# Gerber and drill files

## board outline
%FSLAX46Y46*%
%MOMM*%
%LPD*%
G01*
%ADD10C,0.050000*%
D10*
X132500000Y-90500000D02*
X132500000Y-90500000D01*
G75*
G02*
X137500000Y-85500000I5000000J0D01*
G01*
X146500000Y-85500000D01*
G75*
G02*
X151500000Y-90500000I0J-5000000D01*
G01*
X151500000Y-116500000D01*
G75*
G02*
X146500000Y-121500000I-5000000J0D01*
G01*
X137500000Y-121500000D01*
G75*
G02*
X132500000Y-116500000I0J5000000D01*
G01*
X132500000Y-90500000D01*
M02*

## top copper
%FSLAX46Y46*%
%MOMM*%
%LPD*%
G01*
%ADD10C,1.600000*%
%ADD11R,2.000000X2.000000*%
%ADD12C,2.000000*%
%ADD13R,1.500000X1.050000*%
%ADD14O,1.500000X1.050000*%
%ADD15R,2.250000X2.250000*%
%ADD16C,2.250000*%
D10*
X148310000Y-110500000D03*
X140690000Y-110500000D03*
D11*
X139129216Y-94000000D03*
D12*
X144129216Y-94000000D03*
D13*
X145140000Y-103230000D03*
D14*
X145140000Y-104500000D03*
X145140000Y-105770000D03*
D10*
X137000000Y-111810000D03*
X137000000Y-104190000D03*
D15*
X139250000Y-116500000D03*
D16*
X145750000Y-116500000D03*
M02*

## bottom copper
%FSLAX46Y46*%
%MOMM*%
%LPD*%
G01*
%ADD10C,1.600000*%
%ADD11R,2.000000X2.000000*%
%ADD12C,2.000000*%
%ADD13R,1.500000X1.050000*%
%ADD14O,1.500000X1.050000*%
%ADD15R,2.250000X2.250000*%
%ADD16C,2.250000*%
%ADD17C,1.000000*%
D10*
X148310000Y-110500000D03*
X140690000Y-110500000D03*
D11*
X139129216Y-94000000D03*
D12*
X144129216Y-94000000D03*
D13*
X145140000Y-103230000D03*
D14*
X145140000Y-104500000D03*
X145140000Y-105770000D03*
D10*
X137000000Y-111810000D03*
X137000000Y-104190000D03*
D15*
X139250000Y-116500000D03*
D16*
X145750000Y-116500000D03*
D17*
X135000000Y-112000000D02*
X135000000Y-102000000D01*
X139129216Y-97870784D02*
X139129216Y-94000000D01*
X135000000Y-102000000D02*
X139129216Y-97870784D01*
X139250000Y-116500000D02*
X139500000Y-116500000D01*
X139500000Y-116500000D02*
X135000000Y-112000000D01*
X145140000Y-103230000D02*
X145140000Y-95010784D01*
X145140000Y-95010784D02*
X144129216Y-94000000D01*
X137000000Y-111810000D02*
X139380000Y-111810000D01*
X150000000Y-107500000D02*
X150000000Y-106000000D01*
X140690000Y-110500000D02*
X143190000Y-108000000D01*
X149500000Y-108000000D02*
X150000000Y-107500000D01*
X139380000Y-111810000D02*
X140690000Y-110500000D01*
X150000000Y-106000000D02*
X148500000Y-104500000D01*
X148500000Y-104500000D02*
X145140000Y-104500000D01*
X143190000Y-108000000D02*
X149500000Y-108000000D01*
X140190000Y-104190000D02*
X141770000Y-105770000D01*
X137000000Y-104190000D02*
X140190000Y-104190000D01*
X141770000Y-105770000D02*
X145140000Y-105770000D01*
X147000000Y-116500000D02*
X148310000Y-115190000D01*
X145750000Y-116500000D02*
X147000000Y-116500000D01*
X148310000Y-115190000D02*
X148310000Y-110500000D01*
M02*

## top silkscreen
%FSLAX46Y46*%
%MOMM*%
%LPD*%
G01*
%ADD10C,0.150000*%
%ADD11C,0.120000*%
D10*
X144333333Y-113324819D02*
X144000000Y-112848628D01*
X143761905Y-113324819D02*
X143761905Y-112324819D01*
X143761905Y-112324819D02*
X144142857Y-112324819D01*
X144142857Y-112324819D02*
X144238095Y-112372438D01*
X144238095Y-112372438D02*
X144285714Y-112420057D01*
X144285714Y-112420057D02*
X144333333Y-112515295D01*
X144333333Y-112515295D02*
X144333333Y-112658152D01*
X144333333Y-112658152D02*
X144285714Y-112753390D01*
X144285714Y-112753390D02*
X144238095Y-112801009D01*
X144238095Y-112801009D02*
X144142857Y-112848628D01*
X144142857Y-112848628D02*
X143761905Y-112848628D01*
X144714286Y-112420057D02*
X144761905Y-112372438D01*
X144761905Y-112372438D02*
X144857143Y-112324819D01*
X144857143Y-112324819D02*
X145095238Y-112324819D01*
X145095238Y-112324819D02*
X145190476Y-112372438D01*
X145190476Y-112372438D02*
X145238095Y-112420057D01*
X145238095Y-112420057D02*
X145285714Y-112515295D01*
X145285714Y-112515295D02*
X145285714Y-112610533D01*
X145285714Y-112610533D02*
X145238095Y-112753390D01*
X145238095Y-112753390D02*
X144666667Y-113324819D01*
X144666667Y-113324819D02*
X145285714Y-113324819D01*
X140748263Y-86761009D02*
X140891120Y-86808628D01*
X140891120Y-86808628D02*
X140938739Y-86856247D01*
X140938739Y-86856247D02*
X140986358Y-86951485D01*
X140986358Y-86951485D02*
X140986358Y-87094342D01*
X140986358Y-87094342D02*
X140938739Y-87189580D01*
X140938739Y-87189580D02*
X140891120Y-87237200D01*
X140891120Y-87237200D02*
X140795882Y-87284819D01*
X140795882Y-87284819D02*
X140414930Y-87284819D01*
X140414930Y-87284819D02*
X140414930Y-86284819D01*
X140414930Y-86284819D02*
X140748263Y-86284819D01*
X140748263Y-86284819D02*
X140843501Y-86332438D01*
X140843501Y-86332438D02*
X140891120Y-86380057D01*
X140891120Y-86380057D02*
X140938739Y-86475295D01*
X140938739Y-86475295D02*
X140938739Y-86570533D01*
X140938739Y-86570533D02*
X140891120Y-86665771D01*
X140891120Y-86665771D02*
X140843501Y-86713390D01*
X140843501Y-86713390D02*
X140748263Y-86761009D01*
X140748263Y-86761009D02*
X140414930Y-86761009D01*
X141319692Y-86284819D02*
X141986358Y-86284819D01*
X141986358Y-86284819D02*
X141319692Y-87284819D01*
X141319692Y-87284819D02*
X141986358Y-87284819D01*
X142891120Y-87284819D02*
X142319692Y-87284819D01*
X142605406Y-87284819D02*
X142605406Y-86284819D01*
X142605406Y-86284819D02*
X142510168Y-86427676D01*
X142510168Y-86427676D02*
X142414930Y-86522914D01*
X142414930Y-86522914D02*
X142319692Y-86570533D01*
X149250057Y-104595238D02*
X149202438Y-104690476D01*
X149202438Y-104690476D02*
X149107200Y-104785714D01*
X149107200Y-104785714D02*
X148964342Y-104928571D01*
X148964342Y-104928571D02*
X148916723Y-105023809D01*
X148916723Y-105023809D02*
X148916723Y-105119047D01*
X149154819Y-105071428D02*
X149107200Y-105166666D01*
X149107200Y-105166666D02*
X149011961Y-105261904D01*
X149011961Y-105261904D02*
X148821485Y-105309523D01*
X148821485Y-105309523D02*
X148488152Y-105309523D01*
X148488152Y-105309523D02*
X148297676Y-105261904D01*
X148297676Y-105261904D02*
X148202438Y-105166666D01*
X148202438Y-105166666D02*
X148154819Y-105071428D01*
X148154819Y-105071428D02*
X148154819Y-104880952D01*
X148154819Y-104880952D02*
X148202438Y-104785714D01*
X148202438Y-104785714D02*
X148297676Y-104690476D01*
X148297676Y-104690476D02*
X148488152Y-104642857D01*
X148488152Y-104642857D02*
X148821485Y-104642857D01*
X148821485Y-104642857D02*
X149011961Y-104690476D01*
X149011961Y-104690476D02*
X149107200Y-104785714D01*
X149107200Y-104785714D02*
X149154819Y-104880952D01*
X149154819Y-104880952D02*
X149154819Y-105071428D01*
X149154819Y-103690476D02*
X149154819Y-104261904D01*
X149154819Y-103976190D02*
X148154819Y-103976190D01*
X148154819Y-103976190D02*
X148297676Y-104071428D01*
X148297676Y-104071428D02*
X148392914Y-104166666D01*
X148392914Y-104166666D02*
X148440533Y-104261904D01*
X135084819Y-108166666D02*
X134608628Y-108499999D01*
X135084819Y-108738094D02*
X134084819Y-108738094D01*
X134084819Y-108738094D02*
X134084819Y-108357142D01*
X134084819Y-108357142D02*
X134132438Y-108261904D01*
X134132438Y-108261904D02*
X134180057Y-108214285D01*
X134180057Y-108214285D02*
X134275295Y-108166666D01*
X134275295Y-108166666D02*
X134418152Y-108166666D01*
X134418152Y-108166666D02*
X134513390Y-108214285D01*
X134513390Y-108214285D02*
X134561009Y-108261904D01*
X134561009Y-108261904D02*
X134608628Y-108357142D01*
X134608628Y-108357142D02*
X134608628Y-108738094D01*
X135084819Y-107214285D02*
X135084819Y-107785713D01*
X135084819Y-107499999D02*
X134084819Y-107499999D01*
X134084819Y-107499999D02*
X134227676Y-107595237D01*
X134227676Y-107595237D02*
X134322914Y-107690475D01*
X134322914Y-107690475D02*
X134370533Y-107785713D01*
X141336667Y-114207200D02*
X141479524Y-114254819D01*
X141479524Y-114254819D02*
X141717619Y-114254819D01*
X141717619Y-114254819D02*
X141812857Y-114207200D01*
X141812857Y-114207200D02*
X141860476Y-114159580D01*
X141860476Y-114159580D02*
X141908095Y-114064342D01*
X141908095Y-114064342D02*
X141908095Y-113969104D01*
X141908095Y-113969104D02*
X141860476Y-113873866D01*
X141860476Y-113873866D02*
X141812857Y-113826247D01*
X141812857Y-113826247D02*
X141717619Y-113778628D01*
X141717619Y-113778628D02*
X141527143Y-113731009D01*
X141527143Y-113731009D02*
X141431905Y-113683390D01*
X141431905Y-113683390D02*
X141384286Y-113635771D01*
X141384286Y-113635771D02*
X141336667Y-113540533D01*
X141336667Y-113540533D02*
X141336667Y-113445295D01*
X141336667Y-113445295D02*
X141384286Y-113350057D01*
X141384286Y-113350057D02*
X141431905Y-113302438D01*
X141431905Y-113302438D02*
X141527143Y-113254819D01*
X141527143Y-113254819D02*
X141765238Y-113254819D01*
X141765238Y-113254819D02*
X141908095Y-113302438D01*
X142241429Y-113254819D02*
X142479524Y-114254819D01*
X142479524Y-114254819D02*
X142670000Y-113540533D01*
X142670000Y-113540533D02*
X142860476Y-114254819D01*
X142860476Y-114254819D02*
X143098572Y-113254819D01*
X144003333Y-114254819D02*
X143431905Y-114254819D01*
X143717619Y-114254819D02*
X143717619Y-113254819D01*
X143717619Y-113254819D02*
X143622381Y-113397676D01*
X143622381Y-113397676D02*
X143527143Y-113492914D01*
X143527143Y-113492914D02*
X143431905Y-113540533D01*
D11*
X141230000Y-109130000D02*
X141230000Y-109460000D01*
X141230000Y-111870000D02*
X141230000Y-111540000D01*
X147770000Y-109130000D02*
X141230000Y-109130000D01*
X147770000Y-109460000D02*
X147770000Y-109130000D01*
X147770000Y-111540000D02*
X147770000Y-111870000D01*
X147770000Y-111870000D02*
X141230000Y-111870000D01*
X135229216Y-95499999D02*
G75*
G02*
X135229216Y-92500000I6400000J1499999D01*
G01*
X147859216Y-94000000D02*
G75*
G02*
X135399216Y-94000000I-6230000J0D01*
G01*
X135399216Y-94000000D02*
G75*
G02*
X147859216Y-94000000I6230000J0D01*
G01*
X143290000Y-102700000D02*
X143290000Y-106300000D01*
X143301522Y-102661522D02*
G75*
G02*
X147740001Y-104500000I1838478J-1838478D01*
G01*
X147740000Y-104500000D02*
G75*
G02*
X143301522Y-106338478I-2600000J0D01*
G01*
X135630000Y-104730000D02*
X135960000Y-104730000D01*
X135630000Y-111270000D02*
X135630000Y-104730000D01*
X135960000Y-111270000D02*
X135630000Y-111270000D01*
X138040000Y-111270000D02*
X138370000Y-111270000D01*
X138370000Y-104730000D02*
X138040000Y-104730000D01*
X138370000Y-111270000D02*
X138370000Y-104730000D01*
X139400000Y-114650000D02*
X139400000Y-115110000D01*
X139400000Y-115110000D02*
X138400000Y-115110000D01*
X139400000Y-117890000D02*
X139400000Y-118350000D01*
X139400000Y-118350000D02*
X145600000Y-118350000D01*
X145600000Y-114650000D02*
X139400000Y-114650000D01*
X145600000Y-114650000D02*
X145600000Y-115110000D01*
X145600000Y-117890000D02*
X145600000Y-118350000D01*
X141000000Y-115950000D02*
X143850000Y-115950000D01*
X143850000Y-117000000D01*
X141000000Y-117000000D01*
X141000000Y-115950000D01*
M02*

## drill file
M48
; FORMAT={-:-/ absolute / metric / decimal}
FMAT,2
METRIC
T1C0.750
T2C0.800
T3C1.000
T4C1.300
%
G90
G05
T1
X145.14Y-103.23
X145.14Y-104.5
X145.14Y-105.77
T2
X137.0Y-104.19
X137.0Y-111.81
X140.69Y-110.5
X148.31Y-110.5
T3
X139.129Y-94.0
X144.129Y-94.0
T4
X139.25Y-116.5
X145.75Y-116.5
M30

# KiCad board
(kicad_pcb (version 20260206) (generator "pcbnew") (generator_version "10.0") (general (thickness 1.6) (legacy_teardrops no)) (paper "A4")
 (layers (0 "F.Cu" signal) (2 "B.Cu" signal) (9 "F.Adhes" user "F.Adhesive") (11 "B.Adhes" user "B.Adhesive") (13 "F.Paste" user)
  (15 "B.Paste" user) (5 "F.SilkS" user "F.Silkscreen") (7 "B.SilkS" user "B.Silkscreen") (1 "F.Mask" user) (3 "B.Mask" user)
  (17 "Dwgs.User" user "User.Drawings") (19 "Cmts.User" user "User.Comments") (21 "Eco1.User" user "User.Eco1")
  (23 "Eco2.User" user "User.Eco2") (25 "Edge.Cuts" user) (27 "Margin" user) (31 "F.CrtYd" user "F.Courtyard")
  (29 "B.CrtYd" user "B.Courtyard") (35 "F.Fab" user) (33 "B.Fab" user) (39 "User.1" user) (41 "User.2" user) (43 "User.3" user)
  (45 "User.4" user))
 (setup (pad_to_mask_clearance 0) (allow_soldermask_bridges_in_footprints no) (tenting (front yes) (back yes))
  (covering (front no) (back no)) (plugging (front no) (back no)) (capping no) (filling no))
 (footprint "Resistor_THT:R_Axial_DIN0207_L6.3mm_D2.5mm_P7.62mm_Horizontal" (layer "F.Cu") (at 148.31 110.5 180)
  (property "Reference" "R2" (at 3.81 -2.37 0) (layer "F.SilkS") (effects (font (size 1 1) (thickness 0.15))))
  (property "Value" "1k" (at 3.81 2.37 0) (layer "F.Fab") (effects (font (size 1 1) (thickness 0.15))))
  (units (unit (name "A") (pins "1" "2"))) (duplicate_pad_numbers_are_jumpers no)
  (fp_line (start 7.08 1.37) (end 7.08 1.04) (stroke (width 0.12) (type solid)) (layer "F.SilkS"))
  (fp_line (start 7.08 -1.37) (end 7.08 -1.04) (stroke (width 0.12) (type solid)) (layer "F.SilkS"))
  (fp_line (start 0.54 1.37) (end 7.08 1.37) (stroke (width 0.12) (type solid)) (layer "F.SilkS"))
  (fp_line (start 0.54 1.04) (end 0.54 1.37) (stroke (width 0.12) (type solid)) (layer "F.SilkS"))
  (fp_line (start 0.54 -1.04) (end 0.54 -1.37) (stroke (width 0.12) (type solid)) (layer "F.SilkS"))
  (fp_line (start 0.54 -1.37) (end 7.08 -1.37) (stroke (width 0.12) (type solid)) (layer "F.SilkS"))
  (pad "1" thru_hole circle (at 0 0 180) (size 1.6 1.6) (drill 0.8) (layers "*.Cu" "*.Mask") (remove_unused_layers no) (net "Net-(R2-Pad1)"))
  (pad "2" thru_hole circle (at 7.62 0 180) (size 1.6 1.6) (drill 0.8) (layers "*.Cu" "*.Mask") (remove_unused_layers no) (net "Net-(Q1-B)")))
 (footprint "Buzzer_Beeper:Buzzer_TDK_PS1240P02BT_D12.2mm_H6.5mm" (layer "F.Cu") (at 139.129216 94)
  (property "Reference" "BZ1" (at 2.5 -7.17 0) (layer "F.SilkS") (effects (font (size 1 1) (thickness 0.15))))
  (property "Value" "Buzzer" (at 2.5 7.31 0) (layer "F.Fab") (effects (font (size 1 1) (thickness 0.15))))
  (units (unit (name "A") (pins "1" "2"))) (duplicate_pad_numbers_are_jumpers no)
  (fp_arc (start -3.9 1.499999) (mid -4.073431 0) (end -3.9 -1.5) (stroke (width 0.12) (type solid)) (layer "F.SilkS"))
  (fp_circle (center 2.5 0) (end 8.73 0) (stroke (width 0.12) (type solid)) (fill no) (layer "F.SilkS"))
  (pad "1" thru_hole rect (at 0 0) (size 2 2) (drill 1) (layers "*.Cu" "*.Mask") (remove_unused_layers no) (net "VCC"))
  (pad "2" thru_hole circle (at 5 0) (size 2 2) (drill 1) (layers "*.Cu" "*.Mask") (remove_unused_layers no) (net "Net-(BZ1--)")))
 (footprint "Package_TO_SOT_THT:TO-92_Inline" (layer "F.Cu") (at 145.14 103.23 -90)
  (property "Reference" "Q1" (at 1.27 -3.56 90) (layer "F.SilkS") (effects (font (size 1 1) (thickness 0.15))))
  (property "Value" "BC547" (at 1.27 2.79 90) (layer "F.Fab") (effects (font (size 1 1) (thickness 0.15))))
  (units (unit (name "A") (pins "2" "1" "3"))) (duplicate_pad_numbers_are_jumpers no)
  (fp_line (start -0.53 1.85) (end 3.07 1.85) (stroke (width 0.12) (type solid)) (layer "F.SilkS"))
  (fp_arc (start -0.568478 1.838478) (mid -1.132087 -0.994977) (end 1.27 -2.6) (stroke (width 0.12) (type solid)) (layer "F.SilkS"))
  (fp_arc (start 1.27 -2.6) (mid 3.672087 -0.994977) (end 3.108478 1.838478) (stroke (width 0.12) (type solid)) (layer "F.SilkS"))
  (pad "1" thru_hole rect (at 0 0 270) (size 1.05 1.5) (drill 0.75) (layers "*.Cu" "*.Mask") (remove_unused_layers no) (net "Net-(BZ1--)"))
  (pad "2" thru_hole oval (at 1.27 0 270) (size 1.05 1.5) (drill 0.75) (layers "*.Cu" "*.Mask") (remove_unused_layers no) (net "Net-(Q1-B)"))
  (pad "3" thru_hole oval (at 2.54 0 270) (size 1.05 1.5) (drill 0.75) (layers "*.Cu" "*.Mask") (remove_unused_layers no) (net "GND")))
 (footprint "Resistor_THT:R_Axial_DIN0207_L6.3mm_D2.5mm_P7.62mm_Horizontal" (layer "F.Cu") (at 137 111.81 90)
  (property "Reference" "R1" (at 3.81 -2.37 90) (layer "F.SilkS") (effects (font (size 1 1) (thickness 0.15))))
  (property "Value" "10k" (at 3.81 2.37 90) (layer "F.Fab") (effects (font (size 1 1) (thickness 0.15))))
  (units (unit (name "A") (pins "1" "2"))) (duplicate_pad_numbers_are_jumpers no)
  (fp_line (start 7.08 -1.37) (end 7.08 -1.04) (stroke (width 0.12) (type solid)) (layer "F.SilkS"))
  (fp_line (start 0.54 -1.37) (end 7.08 -1.37) (stroke (width 0.12) (type solid)) (layer "F.SilkS"))
  (fp_line (start 0.54 -1.04) (end 0.54 -1.37) (stroke (width 0.12) (type solid)) (layer "F.SilkS"))
  (fp_line (start 0.54 1.04) (end 0.54 1.37) (stroke (width 0.12) (type solid)) (layer "F.SilkS"))
  (fp_line (start 7.08 1.37) (end 7.08 1.04) (stroke (width 0.12) (type solid)) (layer "F.SilkS"))
  (fp_line (start 0.54 1.37) (end 7.08 1.37) (stroke (width 0.12) (type solid)) (layer "F.SilkS"))
  (pad "1" thru_hole circle (at 0 0 90) (size 1.6 1.6) (drill 0.8) (layers "*.Cu" "*.Mask") (remove_unused_layers no) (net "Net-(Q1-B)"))
  (pad "2" thru_hole circle (at 7.62 0 90) (size 1.6 1.6) (drill 0.8) (layers "*.Cu" "*.Mask") (remove_unused_layers no) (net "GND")))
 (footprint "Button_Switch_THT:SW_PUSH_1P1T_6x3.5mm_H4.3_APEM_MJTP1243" (layer "F.Cu") (at 139.25 116.5)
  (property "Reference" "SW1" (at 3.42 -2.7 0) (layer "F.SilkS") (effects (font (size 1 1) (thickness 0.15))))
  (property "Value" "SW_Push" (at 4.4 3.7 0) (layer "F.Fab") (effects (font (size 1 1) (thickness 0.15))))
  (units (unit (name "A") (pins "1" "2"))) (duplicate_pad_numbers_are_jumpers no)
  (fp_line (start 0.15 -1.85) (end 0.15 -1.39) (stroke (width 0.12) (type default)) (layer "F.SilkS"))
  (fp_line (start 0.15 -1.39) (end -0.85 -1.39) (stroke (width 0.12) (type default)) (layer "F.SilkS"))
  (fp_line (start 0.15 1.39) (end 0.15 1.85) (stroke (width 0.12) (type solid)) (layer "F.SilkS"))
  (fp_line (start 0.15 1.85) (end 6.35 1.85) (stroke (width 0.12) (type solid)) (layer "F.SilkS"))
  (fp_line (start 6.35 -1.85) (end 0.15 -1.85) (stroke (width 0.12) (type solid)) (layer "F.SilkS"))
  (fp_line (start 6.35 -1.85) (end 6.35 -1.39) (stroke (width 0.12) (type solid)) (layer "F.SilkS"))
  (fp_line (start 6.35 1.39) (end 6.35 1.85) (stroke (width 0.12) (type solid)) (layer "F.SilkS"))
  (fp_rect (start 1.75 -0.55) (end 4.6 0.5) (stroke (width 0.12) (type default)) (fill no) (layer "F.SilkS"))
  (pad "1" thru_hole rect (at 0 0 90) (size 2.25 2.25) (drill 1.3) (layers "*.Cu" "*.Mask") (remove_unused_layers no) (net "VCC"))
  (pad "2" thru_hole circle (at 6.5 0 90) (size 2.25 2.25) (drill 1.3) (layers "*.Cu" "*.Mask") (remove_unused_layers no)
   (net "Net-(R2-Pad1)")))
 (gr_rect (start 132.5 85.5) (end 151.5 121.5) (radius 5) (stroke (width 0.05) (type solid)) (fill no) (layer "Edge.Cuts"))
 (segment (start 135 112) (end 135 102) (width 1) (layer "B.Cu") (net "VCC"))
 (segment (start 139.129216 97.870784) (end 139.129216 94) (width 1) (layer "B.Cu") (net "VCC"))
 (segment (start 135 102) (end 139.129216 97.870784) (width 1) (layer "B.Cu") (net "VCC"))
 (segment (start 139.25 116.5) (end 139.5 116.5) (width 1) (layer "B.Cu") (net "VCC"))
 (segment (start 139.5 116.5) (end 135 112) (width 1) (layer "B.Cu") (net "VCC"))
 (segment (start 145.14 103.23) (end 145.14 95.010784) (width 1) (layer "B.Cu") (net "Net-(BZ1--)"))
 (segment (start 145.14 95.010784) (end 144.129216 94) (width 1) (layer "B.Cu") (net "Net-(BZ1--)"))
 (segment (start 137 111.81) (end 139.38 111.81) (width 1) (layer "B.Cu") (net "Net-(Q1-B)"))
 (segment (start 150 107.5) (end 150 106) (width 1) (layer "B.Cu") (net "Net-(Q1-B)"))
 (segment (start 140.69 110.5) (end 143.19 108) (width 1) (layer "B.Cu") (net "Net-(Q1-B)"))
 (segment (start 149.5 108) (end 150 107.5) (width 1) (layer "B.Cu") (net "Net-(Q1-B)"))
 (segment (start 139.38 111.81) (end 140.69 110.5) (width 1) (layer "B.Cu") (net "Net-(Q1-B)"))
 (segment (start 150 106) (end 148.5 104.5) (width 1) (layer "B.Cu") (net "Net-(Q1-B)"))
 (segment (start 148.5 104.5) (end 145.14 104.5) (width 1) (layer "B.Cu") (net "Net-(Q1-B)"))
 (segment (start 143.19 108) (end 149.5 108) (width 1) (layer "B.Cu") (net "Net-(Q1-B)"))
 (segment (start 140.19 104.19) (end 141.77 105.77) (width 1) (layer "B.Cu") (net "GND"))
 (segment (start 137 104.19) (end 140.19 104.19) (width 1) (layer "B.Cu") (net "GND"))
 (segment (start 141.77 105.77) (end 145.14 105.77) (width 1) (layer "B.Cu") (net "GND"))
 (segment (start 147 116.5) (end 148.31 115.19) (width 1) (layer "B.Cu") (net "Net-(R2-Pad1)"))
 (segment (start 145.75 116.5) (end 147 116.5) (width 1) (layer "B.Cu") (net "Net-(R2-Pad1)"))
 (segment (start 148.31 115.19) (end 148.31 110.5) (width 1) (layer "B.Cu") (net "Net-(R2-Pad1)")))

